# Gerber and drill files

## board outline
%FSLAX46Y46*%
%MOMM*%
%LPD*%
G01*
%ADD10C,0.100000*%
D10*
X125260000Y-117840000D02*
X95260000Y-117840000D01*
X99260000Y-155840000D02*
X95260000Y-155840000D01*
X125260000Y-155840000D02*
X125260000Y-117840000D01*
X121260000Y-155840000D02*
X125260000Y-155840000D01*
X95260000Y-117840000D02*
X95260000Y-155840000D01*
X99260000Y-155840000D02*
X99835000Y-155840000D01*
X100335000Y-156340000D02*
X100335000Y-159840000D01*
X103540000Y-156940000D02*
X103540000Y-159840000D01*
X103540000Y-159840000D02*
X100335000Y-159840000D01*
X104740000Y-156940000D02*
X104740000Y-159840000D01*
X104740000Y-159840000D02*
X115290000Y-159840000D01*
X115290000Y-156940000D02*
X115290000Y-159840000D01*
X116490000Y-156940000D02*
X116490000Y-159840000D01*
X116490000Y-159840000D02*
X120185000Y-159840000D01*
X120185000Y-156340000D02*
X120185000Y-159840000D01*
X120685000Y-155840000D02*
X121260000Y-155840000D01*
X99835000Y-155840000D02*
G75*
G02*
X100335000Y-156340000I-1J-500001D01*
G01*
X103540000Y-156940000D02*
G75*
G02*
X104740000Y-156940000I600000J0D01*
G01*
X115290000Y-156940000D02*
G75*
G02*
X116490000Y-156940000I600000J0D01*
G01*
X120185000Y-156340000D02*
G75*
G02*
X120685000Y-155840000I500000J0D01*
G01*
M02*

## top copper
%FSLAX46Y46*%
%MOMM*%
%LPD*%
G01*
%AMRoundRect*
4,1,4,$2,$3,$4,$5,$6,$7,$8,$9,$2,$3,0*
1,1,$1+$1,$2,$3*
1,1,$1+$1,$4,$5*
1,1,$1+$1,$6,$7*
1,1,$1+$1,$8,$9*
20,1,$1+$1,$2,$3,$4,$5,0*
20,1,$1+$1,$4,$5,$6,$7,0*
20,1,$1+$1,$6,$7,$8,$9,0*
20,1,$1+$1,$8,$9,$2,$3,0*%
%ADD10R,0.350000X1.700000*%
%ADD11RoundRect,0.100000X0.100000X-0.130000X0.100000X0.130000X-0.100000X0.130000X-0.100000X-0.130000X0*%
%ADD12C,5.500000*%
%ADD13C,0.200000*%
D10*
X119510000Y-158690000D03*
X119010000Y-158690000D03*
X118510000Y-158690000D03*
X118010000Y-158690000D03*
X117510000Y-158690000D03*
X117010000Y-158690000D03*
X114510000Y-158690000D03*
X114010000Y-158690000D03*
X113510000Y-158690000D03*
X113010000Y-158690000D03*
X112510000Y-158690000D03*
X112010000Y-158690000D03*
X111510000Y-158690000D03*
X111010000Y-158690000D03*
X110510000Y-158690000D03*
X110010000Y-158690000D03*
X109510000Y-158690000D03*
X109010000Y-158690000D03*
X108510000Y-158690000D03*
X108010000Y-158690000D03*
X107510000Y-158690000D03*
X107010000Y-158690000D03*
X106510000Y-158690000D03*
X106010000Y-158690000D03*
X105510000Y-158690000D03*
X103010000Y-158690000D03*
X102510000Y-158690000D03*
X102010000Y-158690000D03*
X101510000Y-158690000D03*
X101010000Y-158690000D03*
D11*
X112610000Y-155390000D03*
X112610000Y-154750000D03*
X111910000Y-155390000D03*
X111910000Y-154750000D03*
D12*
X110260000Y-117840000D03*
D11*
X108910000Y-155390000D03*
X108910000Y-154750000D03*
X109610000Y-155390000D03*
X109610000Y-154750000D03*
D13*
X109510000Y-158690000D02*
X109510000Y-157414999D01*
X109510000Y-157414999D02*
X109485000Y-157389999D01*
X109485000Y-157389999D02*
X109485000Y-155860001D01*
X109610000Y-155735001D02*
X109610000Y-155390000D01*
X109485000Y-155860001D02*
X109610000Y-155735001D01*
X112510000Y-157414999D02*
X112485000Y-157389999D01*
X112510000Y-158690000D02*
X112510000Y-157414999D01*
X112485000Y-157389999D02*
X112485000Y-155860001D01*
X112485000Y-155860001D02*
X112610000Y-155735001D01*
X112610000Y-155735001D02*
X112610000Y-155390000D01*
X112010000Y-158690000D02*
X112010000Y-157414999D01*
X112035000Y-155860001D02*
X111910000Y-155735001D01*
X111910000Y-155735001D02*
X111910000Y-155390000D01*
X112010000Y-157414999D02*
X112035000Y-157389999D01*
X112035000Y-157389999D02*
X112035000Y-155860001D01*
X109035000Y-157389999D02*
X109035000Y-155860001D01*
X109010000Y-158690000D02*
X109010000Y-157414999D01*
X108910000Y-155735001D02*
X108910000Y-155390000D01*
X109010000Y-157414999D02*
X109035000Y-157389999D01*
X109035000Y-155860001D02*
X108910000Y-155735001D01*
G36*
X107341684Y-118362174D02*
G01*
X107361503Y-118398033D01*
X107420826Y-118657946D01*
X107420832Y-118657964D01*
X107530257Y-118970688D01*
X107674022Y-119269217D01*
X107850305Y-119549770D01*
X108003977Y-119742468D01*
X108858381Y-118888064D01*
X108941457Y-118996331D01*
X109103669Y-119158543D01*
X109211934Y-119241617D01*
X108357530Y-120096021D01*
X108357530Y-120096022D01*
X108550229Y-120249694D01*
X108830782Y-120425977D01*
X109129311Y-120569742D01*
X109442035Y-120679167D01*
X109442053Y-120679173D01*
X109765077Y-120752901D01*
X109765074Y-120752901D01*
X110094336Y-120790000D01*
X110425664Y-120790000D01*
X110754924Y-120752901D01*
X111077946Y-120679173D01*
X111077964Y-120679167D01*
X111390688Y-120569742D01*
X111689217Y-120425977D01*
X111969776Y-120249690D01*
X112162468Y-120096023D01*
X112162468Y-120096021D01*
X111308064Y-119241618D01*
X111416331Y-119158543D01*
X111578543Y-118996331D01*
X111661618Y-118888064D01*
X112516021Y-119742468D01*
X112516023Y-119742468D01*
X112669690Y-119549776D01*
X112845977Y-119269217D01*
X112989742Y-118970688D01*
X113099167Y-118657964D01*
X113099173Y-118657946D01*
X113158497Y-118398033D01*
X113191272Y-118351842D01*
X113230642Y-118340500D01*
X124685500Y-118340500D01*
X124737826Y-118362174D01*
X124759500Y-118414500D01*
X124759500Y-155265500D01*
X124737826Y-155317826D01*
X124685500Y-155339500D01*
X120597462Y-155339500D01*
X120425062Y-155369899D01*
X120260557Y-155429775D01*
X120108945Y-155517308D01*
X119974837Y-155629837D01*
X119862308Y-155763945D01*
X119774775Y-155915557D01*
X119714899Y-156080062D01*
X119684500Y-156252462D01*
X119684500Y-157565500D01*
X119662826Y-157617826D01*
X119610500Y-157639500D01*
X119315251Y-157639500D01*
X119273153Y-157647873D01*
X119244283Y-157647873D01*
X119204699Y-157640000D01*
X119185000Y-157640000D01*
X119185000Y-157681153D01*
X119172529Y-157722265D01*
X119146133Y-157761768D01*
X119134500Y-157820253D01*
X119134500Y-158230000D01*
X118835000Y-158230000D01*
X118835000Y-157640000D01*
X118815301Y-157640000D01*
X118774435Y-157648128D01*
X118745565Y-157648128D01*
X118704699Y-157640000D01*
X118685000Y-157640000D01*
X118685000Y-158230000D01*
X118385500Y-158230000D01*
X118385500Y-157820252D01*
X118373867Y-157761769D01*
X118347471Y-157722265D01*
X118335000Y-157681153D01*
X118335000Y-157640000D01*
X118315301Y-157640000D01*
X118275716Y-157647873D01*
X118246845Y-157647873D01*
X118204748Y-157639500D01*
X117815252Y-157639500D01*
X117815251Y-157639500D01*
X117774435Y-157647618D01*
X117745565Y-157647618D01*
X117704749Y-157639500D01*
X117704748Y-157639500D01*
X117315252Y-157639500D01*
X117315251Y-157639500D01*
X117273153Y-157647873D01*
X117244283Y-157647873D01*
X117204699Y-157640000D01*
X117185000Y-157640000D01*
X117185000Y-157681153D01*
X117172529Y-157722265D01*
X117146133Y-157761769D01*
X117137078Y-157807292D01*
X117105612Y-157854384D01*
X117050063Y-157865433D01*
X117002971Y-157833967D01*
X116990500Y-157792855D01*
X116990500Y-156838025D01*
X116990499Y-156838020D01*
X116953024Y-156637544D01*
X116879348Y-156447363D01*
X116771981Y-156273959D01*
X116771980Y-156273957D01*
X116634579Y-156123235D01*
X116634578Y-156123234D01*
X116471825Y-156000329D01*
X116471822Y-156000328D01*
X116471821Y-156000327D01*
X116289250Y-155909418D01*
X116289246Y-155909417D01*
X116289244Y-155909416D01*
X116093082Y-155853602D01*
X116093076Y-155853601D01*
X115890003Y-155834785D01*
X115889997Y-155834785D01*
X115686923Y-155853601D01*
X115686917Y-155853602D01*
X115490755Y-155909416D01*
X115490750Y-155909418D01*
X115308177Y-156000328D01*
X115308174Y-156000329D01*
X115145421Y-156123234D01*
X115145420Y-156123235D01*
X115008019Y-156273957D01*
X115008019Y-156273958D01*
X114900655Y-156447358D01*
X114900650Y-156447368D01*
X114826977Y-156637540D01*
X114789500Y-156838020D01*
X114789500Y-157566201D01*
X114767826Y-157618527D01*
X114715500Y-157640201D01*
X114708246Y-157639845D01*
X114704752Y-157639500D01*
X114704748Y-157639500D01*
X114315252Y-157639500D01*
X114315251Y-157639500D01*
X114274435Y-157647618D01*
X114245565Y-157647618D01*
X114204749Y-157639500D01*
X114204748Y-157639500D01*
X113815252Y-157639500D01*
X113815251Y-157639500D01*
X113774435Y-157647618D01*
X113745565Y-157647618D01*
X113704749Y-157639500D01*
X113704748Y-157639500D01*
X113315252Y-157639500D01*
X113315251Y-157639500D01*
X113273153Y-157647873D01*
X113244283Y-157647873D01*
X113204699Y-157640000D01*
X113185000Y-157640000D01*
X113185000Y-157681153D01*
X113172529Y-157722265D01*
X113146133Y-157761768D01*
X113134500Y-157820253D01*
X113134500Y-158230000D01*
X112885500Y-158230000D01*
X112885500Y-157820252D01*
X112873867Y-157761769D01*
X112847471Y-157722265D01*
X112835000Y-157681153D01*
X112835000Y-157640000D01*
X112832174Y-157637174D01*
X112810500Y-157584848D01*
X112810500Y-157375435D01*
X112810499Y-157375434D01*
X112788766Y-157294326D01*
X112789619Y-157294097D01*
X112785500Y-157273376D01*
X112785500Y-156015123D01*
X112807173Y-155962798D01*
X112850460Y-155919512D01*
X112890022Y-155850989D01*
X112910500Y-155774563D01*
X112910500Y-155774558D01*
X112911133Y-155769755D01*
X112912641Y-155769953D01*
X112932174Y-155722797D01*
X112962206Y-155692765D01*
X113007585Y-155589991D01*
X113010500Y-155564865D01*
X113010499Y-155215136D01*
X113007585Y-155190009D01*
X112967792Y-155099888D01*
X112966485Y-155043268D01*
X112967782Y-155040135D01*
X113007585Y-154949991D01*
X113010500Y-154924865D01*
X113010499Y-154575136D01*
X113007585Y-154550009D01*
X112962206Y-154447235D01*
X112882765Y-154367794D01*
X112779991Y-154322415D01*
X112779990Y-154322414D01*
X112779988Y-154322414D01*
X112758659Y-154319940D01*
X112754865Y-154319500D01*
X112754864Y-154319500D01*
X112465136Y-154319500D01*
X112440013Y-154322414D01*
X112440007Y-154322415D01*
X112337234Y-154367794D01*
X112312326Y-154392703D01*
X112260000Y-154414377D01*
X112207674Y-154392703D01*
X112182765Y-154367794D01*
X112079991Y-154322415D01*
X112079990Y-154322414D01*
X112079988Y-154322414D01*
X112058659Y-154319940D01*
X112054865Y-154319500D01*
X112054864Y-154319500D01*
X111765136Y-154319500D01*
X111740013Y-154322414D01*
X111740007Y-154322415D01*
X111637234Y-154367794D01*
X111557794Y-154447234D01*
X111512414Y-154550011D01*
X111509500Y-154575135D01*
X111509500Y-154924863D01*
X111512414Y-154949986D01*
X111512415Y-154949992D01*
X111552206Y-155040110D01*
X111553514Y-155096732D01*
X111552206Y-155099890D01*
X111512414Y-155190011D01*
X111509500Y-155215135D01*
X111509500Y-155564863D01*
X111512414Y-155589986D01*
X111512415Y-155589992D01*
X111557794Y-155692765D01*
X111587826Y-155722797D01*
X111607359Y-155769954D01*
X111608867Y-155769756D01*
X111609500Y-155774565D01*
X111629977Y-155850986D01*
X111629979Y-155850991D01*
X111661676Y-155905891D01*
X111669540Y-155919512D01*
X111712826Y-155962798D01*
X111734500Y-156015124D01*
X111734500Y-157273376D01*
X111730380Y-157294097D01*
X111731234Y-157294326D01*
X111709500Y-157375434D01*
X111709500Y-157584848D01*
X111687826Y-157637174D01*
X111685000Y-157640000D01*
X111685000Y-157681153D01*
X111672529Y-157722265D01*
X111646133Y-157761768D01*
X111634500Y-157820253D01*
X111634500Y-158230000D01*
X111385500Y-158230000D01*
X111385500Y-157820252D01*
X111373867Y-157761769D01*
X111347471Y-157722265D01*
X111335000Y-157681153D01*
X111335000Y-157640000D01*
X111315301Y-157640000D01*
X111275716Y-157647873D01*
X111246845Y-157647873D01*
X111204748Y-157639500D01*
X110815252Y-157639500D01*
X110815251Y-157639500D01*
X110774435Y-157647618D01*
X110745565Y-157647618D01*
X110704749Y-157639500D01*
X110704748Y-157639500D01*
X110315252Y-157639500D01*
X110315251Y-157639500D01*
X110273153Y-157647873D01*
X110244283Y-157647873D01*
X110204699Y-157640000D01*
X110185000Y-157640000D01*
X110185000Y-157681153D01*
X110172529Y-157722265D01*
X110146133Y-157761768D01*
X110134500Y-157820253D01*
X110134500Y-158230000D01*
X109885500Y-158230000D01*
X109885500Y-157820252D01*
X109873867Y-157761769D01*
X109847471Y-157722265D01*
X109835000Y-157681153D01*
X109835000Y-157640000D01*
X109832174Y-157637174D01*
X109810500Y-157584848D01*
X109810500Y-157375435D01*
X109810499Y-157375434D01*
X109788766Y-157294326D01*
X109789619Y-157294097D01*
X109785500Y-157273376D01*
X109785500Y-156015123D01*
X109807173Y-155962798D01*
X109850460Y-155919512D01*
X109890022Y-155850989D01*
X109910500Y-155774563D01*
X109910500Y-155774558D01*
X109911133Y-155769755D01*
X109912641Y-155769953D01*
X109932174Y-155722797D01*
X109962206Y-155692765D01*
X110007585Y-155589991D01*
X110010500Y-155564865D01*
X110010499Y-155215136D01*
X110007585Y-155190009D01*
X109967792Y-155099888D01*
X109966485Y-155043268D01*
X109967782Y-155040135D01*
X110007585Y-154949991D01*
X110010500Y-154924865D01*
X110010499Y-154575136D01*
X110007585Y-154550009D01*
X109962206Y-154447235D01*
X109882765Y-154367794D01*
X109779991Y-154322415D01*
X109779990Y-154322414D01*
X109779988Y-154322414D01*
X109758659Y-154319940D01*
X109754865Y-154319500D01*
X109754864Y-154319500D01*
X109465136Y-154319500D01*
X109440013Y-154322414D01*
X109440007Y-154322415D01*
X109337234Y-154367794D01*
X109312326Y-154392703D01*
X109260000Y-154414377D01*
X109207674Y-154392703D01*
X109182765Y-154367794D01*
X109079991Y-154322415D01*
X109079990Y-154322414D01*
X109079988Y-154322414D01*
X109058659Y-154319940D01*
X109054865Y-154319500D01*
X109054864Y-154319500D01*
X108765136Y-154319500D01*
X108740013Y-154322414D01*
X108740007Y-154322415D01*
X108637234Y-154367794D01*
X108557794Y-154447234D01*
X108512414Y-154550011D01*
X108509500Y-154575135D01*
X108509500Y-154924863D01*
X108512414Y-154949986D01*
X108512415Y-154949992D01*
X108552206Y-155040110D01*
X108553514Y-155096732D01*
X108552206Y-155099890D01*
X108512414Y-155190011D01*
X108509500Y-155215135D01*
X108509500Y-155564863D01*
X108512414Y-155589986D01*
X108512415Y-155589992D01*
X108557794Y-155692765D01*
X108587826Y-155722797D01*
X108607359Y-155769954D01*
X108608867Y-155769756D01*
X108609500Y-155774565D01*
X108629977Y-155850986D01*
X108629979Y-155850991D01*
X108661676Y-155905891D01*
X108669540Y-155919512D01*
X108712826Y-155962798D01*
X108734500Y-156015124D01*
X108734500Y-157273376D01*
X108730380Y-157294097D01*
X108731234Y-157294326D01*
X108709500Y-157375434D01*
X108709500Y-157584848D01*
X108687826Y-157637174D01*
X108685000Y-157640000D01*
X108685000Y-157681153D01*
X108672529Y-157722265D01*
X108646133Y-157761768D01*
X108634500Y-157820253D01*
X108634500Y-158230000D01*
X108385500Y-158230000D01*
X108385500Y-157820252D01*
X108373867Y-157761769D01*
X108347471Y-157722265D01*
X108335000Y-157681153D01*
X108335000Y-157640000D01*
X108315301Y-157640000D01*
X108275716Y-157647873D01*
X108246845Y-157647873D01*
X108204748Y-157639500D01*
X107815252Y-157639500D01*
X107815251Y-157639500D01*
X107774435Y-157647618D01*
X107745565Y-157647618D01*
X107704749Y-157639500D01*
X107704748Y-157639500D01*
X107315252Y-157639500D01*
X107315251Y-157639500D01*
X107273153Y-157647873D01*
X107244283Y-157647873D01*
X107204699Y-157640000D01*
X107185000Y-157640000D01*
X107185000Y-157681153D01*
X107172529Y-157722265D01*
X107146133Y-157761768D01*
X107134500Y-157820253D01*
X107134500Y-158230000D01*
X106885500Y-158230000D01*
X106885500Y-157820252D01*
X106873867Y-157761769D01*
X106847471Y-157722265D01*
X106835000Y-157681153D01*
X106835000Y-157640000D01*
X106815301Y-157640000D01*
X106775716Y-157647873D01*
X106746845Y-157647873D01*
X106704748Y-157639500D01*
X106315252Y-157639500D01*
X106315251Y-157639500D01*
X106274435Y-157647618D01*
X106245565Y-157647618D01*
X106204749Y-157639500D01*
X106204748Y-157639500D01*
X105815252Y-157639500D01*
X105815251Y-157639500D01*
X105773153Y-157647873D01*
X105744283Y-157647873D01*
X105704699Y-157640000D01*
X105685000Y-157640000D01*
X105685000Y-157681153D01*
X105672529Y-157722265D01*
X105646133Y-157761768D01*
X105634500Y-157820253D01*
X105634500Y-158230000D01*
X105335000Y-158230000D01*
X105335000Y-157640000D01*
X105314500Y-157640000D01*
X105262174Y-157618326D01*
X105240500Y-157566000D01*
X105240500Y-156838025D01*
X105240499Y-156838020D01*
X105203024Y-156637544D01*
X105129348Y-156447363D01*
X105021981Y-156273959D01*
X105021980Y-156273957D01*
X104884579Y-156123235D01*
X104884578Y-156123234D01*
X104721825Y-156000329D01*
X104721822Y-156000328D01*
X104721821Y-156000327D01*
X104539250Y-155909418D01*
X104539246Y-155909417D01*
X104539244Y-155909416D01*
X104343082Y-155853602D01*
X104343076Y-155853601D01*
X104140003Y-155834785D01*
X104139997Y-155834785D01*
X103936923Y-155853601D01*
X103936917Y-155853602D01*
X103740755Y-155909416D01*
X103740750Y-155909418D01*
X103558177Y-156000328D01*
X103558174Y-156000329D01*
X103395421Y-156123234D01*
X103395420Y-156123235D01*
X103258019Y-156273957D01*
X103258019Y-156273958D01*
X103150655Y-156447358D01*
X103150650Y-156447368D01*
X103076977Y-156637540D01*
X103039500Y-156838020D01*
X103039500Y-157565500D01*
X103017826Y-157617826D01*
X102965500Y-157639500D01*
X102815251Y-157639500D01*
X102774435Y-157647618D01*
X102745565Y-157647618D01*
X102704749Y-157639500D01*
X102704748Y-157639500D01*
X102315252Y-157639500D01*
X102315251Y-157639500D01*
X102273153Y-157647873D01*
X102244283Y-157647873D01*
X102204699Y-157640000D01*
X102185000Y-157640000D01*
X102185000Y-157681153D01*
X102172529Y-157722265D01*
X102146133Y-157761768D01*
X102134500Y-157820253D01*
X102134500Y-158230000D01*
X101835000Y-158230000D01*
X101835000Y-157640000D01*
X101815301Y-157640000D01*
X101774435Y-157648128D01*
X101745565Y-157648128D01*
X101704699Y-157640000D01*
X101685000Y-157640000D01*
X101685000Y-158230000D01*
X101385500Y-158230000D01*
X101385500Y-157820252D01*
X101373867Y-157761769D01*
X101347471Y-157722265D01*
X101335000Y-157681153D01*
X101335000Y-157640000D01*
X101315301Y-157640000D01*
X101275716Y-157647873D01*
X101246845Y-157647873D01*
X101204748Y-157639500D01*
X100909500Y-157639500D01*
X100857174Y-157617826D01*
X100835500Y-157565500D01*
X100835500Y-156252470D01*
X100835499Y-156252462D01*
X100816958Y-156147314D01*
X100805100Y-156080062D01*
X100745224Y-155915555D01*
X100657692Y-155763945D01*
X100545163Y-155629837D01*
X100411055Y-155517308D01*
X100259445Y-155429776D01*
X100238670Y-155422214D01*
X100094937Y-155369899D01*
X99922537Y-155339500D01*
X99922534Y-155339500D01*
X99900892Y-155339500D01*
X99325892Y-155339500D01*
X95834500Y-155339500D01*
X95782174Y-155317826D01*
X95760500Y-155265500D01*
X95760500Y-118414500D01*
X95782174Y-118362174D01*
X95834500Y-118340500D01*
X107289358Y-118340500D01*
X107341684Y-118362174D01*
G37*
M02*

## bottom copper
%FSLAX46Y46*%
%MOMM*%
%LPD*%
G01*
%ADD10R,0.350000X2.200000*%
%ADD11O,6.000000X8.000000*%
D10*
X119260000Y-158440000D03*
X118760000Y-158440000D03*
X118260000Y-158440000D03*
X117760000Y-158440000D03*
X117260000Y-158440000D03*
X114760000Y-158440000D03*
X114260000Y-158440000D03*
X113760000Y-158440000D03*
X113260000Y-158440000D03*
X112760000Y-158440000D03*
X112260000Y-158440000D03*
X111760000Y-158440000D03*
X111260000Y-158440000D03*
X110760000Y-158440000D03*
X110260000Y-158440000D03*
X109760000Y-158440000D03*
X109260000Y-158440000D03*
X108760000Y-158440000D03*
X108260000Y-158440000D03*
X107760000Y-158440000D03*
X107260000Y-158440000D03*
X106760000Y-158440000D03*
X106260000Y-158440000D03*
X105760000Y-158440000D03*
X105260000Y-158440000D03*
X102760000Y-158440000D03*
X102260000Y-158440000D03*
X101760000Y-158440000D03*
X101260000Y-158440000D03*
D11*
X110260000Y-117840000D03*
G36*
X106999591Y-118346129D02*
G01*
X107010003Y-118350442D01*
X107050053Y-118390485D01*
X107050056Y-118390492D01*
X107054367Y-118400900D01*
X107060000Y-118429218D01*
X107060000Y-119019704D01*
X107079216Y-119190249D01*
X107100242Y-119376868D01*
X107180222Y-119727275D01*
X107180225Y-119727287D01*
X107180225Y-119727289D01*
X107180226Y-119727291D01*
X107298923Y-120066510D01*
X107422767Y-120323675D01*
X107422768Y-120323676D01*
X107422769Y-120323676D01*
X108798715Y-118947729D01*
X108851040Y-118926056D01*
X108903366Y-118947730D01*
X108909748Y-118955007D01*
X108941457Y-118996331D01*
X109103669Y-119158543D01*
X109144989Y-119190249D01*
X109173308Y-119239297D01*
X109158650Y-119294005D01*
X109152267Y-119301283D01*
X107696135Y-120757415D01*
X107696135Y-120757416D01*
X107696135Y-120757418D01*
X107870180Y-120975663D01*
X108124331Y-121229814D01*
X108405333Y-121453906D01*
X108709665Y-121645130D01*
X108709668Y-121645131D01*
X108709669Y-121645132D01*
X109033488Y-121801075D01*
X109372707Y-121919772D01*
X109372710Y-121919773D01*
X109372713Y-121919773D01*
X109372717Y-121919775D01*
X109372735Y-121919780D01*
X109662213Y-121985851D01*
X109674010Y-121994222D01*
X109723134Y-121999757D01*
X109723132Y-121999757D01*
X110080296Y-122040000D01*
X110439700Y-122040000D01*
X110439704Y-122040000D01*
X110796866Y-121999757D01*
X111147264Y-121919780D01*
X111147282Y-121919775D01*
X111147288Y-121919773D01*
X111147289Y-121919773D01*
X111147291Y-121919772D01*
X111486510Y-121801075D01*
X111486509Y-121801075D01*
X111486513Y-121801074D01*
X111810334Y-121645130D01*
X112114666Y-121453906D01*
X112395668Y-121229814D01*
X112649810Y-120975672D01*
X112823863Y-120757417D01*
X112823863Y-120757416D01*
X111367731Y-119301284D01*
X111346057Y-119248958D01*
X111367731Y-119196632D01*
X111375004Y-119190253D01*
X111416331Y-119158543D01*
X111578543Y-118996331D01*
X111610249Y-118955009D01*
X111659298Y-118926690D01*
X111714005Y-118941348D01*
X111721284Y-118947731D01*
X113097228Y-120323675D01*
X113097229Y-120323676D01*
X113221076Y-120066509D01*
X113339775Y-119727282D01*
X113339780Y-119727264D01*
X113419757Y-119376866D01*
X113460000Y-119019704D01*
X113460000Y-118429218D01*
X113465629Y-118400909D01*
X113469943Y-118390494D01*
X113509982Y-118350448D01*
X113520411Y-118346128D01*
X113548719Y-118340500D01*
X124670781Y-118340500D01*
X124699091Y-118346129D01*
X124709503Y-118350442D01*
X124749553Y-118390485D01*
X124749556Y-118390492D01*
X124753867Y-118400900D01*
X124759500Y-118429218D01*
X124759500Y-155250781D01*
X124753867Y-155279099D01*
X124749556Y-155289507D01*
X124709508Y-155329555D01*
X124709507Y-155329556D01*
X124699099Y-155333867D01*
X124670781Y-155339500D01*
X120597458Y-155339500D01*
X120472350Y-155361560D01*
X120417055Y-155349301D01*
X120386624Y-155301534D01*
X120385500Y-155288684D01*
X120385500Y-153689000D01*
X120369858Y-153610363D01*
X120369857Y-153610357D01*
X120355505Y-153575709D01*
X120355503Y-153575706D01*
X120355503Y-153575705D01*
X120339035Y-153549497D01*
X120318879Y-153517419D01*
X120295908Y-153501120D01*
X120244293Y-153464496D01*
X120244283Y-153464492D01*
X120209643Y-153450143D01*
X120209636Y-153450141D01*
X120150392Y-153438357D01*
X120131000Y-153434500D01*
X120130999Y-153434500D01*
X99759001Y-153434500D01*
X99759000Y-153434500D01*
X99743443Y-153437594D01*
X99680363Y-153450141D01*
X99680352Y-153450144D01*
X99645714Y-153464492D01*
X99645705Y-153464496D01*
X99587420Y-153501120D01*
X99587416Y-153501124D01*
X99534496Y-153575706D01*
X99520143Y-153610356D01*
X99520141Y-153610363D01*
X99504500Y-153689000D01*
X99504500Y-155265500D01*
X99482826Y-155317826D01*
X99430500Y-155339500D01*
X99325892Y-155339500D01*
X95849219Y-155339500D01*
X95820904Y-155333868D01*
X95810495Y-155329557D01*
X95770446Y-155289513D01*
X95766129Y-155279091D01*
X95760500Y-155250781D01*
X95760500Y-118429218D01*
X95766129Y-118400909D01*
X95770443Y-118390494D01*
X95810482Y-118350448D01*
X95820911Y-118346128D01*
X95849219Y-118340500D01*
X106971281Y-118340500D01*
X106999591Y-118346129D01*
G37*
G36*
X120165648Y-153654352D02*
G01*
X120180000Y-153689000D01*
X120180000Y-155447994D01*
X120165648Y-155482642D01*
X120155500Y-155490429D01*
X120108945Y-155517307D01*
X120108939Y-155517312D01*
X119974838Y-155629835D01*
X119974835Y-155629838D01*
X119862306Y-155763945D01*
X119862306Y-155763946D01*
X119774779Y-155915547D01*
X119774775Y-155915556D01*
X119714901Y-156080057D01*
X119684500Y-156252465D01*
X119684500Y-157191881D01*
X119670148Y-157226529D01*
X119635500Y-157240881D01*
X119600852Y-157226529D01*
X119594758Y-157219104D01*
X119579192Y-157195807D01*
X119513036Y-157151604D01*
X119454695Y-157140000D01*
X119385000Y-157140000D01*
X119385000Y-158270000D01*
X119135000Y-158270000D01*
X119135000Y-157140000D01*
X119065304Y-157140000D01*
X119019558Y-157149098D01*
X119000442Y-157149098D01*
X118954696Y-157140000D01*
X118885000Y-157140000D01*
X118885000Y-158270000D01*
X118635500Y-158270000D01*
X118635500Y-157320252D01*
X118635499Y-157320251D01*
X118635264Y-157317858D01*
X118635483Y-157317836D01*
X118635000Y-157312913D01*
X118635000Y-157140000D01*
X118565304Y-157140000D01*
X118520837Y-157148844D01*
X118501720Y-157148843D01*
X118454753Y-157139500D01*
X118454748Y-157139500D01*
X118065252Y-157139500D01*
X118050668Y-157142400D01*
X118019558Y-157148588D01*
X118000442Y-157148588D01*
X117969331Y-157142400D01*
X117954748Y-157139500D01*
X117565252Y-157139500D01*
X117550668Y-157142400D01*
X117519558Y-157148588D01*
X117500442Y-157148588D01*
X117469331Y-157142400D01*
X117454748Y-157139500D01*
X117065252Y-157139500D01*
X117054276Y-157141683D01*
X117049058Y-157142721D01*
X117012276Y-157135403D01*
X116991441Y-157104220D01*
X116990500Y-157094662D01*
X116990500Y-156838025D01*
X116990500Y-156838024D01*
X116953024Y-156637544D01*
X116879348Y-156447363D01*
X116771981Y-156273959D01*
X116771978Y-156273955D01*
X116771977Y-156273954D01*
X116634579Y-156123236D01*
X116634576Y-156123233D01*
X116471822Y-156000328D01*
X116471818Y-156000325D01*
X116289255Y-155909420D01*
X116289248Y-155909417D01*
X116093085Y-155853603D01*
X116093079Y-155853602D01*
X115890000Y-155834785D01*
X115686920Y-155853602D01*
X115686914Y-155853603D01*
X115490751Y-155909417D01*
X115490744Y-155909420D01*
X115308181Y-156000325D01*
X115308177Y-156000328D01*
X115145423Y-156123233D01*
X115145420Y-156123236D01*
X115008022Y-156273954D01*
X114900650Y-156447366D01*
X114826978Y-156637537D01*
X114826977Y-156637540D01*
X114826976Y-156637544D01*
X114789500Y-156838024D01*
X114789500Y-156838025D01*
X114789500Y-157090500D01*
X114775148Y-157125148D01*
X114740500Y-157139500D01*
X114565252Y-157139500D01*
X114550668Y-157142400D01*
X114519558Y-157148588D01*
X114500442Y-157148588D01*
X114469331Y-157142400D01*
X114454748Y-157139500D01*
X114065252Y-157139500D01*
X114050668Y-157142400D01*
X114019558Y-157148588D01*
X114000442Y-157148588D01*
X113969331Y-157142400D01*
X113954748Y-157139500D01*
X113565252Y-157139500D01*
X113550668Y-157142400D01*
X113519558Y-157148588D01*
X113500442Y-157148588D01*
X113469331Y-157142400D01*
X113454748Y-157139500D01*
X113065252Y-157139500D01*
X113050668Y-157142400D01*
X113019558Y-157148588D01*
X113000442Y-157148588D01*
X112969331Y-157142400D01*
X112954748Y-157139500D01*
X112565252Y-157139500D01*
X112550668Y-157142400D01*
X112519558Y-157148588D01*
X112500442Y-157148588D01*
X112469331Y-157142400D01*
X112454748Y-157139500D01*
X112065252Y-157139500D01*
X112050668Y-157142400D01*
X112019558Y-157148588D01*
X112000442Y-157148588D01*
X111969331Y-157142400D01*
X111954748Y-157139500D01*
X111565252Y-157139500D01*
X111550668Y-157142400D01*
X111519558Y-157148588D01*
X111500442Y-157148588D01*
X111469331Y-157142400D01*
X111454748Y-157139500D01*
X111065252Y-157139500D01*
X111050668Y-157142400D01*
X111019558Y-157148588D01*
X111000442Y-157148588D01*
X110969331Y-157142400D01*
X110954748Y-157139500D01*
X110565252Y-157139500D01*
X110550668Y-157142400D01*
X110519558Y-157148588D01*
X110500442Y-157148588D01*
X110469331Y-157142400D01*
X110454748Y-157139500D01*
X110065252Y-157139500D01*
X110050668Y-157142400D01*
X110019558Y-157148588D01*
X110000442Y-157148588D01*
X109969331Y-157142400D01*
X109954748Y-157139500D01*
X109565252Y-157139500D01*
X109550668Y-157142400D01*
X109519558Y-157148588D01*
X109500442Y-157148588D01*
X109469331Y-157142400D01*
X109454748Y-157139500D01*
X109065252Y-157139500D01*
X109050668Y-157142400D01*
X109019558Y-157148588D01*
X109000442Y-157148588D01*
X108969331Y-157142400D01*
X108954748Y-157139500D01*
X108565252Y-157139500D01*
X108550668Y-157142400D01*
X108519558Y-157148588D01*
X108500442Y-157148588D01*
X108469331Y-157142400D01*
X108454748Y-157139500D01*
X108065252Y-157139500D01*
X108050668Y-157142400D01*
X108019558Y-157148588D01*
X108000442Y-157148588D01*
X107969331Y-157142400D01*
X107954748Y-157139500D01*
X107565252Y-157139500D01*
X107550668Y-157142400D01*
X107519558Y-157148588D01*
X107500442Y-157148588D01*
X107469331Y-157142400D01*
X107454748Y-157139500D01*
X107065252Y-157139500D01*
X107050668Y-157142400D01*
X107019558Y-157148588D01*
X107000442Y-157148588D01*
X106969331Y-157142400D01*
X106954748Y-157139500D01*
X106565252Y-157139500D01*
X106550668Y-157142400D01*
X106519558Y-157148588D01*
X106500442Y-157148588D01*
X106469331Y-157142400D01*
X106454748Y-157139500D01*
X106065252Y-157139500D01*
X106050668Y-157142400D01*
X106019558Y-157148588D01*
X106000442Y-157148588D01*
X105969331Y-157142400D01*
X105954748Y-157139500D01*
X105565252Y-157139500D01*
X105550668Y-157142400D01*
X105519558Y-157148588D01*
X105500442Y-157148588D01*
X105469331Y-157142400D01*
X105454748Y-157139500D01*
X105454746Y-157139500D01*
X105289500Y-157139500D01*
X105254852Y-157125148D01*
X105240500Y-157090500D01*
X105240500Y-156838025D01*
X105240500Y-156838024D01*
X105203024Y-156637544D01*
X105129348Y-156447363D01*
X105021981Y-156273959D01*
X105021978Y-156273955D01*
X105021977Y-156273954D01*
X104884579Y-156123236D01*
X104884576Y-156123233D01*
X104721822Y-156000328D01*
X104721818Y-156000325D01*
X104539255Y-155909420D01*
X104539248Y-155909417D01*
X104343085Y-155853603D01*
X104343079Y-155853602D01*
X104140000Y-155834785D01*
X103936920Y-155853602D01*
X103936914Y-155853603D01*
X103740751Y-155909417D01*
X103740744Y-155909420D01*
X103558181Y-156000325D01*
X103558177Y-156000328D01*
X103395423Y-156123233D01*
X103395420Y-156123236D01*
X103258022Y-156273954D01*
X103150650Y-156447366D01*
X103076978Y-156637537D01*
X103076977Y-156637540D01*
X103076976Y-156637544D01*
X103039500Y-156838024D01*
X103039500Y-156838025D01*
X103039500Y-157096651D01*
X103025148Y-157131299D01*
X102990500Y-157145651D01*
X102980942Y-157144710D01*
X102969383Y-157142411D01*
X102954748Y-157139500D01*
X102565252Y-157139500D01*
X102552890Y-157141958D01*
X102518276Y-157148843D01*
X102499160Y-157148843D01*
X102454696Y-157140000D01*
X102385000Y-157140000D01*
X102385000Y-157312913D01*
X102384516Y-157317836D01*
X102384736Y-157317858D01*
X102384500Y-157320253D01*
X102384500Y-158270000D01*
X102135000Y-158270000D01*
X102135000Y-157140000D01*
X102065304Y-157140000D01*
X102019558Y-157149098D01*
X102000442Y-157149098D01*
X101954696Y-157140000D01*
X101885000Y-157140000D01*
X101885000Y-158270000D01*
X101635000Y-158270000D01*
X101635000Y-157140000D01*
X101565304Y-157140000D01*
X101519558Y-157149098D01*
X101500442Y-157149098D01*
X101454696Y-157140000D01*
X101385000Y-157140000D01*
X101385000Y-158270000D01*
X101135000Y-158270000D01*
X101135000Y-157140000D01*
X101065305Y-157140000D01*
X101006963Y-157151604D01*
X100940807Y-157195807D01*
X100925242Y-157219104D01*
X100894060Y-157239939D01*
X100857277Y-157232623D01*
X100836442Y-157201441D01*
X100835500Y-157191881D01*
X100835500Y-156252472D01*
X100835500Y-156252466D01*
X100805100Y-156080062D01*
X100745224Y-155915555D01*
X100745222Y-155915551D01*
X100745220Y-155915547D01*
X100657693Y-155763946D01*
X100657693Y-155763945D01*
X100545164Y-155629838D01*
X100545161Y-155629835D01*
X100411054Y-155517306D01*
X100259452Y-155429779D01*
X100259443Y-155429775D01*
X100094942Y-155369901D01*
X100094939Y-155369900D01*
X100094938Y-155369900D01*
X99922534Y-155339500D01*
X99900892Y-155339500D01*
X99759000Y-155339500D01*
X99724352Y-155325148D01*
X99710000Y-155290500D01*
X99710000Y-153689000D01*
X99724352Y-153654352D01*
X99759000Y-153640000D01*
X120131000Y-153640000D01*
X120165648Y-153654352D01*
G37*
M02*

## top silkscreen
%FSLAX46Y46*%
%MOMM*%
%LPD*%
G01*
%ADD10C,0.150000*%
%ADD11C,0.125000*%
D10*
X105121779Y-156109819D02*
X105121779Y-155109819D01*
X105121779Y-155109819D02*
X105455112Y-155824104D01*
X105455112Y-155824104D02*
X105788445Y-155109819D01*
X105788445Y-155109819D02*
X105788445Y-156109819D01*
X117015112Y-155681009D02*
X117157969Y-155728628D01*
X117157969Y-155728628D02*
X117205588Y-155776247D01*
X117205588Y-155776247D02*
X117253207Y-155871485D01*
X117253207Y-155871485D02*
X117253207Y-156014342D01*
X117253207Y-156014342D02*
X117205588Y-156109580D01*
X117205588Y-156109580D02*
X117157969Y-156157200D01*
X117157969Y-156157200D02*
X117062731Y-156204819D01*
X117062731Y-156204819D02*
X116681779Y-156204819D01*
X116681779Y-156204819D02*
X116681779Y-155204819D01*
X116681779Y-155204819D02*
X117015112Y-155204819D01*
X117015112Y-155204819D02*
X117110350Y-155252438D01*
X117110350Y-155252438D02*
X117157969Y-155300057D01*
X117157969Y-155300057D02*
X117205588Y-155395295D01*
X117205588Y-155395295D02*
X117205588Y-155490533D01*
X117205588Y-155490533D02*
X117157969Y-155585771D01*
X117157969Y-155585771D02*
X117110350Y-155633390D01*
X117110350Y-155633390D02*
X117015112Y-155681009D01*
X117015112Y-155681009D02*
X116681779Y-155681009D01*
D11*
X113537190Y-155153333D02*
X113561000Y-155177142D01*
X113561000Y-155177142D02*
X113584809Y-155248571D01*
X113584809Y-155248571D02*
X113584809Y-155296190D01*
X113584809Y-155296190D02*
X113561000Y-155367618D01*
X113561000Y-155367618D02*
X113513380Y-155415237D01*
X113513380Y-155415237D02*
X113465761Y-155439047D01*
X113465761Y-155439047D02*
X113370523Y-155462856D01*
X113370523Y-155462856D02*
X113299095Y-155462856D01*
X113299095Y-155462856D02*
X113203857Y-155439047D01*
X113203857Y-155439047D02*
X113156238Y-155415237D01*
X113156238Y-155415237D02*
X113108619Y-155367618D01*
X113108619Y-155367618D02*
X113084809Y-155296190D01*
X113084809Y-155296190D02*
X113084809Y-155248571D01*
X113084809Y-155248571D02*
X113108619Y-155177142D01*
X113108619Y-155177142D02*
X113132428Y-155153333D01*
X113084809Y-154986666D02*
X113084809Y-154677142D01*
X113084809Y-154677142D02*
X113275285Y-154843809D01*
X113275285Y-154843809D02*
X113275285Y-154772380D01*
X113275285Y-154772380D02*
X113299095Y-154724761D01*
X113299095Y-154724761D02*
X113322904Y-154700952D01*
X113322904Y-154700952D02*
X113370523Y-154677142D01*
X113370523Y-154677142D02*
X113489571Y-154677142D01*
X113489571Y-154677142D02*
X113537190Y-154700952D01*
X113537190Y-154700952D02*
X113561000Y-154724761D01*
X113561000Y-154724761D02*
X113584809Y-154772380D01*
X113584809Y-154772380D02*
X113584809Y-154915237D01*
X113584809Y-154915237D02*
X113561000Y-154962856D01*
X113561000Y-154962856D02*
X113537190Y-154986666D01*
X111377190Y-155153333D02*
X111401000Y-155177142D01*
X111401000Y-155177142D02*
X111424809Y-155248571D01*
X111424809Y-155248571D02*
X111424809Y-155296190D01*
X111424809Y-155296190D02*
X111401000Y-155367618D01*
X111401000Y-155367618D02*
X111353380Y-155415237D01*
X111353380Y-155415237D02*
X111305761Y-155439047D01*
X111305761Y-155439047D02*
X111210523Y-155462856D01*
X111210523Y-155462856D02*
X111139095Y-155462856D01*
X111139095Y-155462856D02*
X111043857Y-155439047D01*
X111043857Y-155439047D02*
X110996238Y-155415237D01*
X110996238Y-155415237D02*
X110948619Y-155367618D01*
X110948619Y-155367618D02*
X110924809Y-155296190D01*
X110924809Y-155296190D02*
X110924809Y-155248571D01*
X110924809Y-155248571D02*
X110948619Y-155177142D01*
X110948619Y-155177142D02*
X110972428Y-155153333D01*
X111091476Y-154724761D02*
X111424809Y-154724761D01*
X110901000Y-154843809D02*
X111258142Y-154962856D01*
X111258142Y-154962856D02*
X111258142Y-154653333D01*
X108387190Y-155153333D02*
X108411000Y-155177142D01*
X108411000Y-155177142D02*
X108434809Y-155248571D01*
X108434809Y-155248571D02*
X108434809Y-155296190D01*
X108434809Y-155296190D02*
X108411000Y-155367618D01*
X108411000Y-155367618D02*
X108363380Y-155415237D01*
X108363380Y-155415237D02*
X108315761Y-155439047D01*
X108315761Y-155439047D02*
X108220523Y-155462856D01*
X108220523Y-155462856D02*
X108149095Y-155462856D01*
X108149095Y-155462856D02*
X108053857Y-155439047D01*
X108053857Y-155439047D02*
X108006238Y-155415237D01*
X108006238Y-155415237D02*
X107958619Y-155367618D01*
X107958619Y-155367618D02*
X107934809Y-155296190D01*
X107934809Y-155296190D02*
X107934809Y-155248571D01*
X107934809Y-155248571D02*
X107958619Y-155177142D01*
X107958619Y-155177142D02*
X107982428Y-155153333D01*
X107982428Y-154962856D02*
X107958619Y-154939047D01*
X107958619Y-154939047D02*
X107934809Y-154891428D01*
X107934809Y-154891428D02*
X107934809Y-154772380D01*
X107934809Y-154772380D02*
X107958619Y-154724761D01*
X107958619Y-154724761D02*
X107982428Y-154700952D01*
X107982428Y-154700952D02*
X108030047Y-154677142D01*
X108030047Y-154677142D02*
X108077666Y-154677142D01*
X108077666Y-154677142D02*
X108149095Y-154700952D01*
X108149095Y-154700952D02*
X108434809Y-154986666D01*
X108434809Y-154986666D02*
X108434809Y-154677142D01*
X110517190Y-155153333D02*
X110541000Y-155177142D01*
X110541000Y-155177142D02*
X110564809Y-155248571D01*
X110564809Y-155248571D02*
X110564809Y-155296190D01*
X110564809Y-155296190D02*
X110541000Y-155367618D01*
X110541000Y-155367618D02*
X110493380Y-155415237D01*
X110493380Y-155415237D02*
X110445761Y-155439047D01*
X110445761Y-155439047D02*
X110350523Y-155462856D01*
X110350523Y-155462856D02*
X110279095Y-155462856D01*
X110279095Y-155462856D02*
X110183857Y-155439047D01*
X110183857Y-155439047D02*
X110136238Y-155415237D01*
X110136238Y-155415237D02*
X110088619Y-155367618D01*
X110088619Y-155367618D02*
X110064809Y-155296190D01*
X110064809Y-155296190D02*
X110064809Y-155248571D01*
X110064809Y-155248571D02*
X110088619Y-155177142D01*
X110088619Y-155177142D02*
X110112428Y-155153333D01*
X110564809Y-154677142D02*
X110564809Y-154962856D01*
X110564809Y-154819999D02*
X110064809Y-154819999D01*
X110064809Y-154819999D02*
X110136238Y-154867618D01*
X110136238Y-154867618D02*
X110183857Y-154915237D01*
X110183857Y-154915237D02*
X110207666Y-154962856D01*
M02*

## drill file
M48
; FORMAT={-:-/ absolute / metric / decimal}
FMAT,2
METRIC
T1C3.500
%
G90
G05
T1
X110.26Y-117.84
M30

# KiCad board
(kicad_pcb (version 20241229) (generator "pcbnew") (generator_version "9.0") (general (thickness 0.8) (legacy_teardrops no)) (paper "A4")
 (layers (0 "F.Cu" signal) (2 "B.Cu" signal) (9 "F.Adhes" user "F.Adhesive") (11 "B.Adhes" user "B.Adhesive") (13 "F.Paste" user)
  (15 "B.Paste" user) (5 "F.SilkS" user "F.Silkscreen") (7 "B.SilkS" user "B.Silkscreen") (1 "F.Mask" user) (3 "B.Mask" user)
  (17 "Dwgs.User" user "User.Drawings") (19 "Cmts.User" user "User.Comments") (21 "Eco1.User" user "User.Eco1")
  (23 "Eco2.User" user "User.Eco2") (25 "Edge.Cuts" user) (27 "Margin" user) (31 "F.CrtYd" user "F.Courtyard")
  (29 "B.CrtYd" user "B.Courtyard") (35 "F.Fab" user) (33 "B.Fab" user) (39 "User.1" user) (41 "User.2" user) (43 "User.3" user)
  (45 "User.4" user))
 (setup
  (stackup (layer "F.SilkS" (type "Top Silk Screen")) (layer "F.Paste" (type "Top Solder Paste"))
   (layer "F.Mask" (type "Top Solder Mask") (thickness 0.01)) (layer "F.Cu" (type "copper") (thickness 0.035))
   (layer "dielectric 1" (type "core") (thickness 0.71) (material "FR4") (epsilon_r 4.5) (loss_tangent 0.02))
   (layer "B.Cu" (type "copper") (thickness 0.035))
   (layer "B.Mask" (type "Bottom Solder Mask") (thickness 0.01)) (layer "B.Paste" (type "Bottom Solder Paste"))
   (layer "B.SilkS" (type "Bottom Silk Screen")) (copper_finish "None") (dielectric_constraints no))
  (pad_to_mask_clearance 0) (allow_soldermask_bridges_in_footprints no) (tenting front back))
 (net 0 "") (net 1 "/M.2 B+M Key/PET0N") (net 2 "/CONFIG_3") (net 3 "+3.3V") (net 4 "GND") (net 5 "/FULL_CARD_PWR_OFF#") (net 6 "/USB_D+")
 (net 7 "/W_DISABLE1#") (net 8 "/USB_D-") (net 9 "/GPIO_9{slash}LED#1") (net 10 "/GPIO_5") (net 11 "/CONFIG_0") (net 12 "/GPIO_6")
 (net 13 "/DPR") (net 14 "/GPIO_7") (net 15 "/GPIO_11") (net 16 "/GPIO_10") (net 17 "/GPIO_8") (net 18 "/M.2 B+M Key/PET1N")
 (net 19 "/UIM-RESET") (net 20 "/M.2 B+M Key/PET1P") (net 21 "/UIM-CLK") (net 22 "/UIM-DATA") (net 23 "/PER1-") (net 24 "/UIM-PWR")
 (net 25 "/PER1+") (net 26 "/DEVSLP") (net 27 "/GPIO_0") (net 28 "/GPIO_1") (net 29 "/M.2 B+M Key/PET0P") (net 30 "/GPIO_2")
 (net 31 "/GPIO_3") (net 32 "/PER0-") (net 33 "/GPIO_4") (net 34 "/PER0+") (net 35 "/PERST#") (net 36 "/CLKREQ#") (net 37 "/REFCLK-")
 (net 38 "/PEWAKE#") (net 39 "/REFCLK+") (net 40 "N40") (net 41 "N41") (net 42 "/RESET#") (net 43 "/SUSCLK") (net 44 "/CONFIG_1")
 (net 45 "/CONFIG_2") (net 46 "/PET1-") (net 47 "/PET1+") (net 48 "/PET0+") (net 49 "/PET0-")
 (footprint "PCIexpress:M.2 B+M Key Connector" (layer "F.Cu") (at 110.26 158.73)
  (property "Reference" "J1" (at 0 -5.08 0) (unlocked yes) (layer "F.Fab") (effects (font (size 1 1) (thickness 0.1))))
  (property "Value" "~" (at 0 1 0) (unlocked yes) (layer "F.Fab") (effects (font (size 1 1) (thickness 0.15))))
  (fp_line (start -11 -2.89) (end -10.425 -2.89) (stroke (width 0.1) (type default)) (layer "Edge.Cuts") (net 1))
  (fp_line (start -9.925 -2.39) (end -9.925 1.11) (stroke (width 0.1) (type default)) (layer "Edge.Cuts") (net 1))
  (fp_line (start -6.72 -1.79) (end -6.72 1.11) (stroke (width 0.1) (type default)) (layer "Edge.Cuts") (net 1))
  (fp_line (start -6.72 1.11) (end -9.925 1.11) (stroke (width 0.1) (type default)) (layer "Edge.Cuts") (net 1))
  (fp_line (start -5.52 -1.79) (end -5.52 1.11) (stroke (width 0.1) (type default)) (layer "Edge.Cuts") (net 1))
  (fp_line (start -5.52 1.11) (end 5.03 1.11) (stroke (width 0.1) (type default)) (layer "Edge.Cuts") (net 1))
  (fp_line (start 5.03 -1.79) (end 5.03 1.11) (stroke (width 0.1) (type default)) (layer "Edge.Cuts") (net 1))
  (fp_line (start 6.23 -1.79) (end 6.23 1.11) (stroke (width 0.1) (type default)) (layer "Edge.Cuts") (net 1))
  (fp_line (start 6.23 1.11) (end 9.925 1.11) (stroke (width 0.1) (type default)) (layer "Edge.Cuts") (net 1))
  (fp_line (start 9.925 -2.39) (end 9.925 1.11) (stroke (width 0.1) (type default)) (layer "Edge.Cuts") (net 1))
  (fp_line (start 10.425 -2.89) (end 11 -2.89) (stroke (width 0.1) (type default)) (layer "Edge.Cuts") (net 1))
  (fp_arc (start -10.425 -2.89) (mid -10.071447 -2.743553) (end -9.925 -2.39) (stroke (width 0.1) (type default)) (layer "Edge.Cuts")
   (net 1))
  (fp_arc (start -6.72 -1.79) (mid -6.12 -2.39) (end -5.52 -1.79) (stroke (width 0.1) (type default)) (layer "Edge.Cuts") (net 1))
  (fp_arc (start 5.03 -1.79) (mid 5.63 -2.39) (end 6.23 -1.79) (stroke (width 0.1) (type default)) (layer "Edge.Cuts") (net 1))
  (fp_arc (start 9.925 -2.39) (mid 10.071447 -2.743553) (end 10.425 -2.89) (stroke (width 0.1) (type default)) (layer "Edge.Cuts") (net 1))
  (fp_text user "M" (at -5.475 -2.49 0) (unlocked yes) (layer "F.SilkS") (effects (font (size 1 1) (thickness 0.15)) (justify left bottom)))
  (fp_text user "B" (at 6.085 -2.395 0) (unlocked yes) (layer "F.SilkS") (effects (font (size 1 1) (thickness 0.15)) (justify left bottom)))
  (pad "1" smd rect (at 9.25 -0.04 180) (size 0.35 1.7) (layers "F.Cu") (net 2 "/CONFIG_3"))
  (pad "2" smd rect (at 9 -0.29 180) (size 0.35 2.2) (layers "B.Cu") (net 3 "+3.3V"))
  (pad "3" smd rect (at 8.75 -0.04 180) (size 0.35 1.7) (layers "F.Cu") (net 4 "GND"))
  (pad "4" smd rect (at 8.5 -0.29 180) (size 0.35 2.2) (layers "B.Cu") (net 3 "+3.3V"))
  (pad "5" smd rect (at 8.25 -0.04 180) (size 0.35 1.7) (layers "F.Cu") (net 4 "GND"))
  (pad "6" smd rect (at 8 -0.29 180) (size 0.35 2.2) (layers "B.Cu") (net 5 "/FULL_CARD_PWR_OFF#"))
  (pad "7" smd rect (at 7.75 -0.04 180) (size 0.35 1.7) (layers "F.Cu") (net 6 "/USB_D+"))
  (pad "8" smd rect (at 7.5 -0.29 180) (size 0.35 2.2) (layers "B.Cu") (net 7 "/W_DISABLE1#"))
  (pad "9" smd rect (at 7.25 -0.04 180) (size 0.35 1.7) (layers "F.Cu") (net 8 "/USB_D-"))
  (pad "10" smd rect (at 7 -0.29 180) (size 0.35 2.2) (layers "B.Cu") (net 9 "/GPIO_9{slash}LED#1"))
  (pad "11" smd rect (at 6.75 -0.04 180) (size 0.35 1.7) (layers "F.Cu") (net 4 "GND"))
  (pad "20" smd rect (at 4.5 -0.29 180) (size 0.35 2.2) (layers "B.Cu") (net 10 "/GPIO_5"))
  (pad "21" smd rect (at 4.25 -0.04 180) (size 0.35 1.7) (layers "F.Cu") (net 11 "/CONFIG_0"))
  (pad "22" smd rect (at 4 -0.29 180) (size 0.35 2.2) (layers "B.Cu") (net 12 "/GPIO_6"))
  (pad "23" smd rect (at 3.75 -0.04 180) (size 0.35 1.7) (layers "F.Cu") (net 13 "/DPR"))
  (pad "24" smd rect (at 3.5 -0.29 180) (size 0.35 2.2) (layers "B.Cu") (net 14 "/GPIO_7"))
  (pad "25" smd rect (at 3.25 -0.04 180) (size 0.35 1.7) (layers "F.Cu") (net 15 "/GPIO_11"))
  (pad "26" smd rect (at 3 -0.29 180) (size 0.35 2.2) (layers "B.Cu") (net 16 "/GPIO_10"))
  (pad "27" smd rect (at 2.75 -0.04 180) (size 0.35 1.7) (layers "F.Cu") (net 4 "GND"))
  (pad "28" smd rect (at 2.5 -0.29 180) (size 0.35 2.2) (layers "B.Cu") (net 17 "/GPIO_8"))
  (pad "29" smd rect (at 2.25 -0.04 180) (size 0.35 1.7) (layers "F.Cu") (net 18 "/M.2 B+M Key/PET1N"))
  (pad "30" smd rect (at 2 -0.29 180) (size 0.35 2.2) (layers "B.Cu") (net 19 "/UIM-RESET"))
  (pad "31" smd rect (at 1.75 -0.04 180) (size 0.35 1.7) (layers "F.Cu") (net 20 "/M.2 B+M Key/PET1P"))
  (pad "32" smd rect (at 1.5 -0.29 180) (size 0.35 2.2) (layers "B.Cu") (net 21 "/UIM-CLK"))
  (pad "33" smd rect (at 1.25 -0.04 180) (size 0.35 1.7) (layers "F.Cu") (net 4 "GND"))
  (pad "34" smd rect (at 1 -0.29 180) (size 0.35 2.2) (layers "B.Cu") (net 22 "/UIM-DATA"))
  (pad "35" smd rect (at 0.75 -0.04 180) (size 0.35 1.7) (layers "F.Cu") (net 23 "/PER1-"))
  (pad "36" smd rect (at 0.5 -0.29 180) (size 0.35 2.2) (layers "B.Cu") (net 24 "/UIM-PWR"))
  (pad "37" smd rect (at 0.25 -0.04 180) (size 0.35 1.7) (layers "F.Cu") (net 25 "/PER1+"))
  (pad "38" smd rect (at 0 -0.29 180) (size 0.35 2.2) (layers "B.Cu") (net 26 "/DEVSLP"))
  (pad "39" smd rect (at -0.25 -0.04 180) (size 0.35 1.7) (layers "F.Cu") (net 4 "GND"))
  (pad "40" smd rect (at -0.5 -0.29 180) (size 0.35 2.2) (layers "B.Cu") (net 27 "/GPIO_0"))
  (pad "41" smd rect (at -0.75 -0.04 180) (size 0.35 1.7) (layers "F.Cu") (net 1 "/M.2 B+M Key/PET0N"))
  (pad "42" smd rect (at -1 -0.29 180) (size 0.35 2.2) (layers "B.Cu") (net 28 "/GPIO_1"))
  (pad "43" smd rect (at -1.25 -0.04 180) (size 0.35 1.7) (layers "F.Cu") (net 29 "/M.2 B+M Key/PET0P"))
  (pad "44" smd rect (at -1.5 -0.29 180) (size 0.35 2.2) (layers "B.Cu") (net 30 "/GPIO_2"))
  (pad "45" smd rect (at -1.75 -0.04 180) (size 0.35 1.7) (layers "F.Cu") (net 4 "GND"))
  (pad "46" smd rect (at -2 -0.29 180) (size 0.35 2.2) (layers "B.Cu") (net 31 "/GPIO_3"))
  (pad "47" smd rect (at -2.25 -0.04 180) (size 0.35 1.7) (layers "F.Cu") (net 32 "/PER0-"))
  (pad "48" smd rect (at -2.5 -0.29 180) (size 0.35 2.2) (layers "B.Cu") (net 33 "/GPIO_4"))
  (pad "49" smd rect (at -2.75 -0.04 180) (size 0.35 1.7) (layers "F.Cu") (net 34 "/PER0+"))
  (pad "50" smd rect (at -3 -0.29 180) (size 0.35 2.2) (layers "B.Cu") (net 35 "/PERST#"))
  (pad "51" smd rect (at -3.25 -0.04 180) (size 0.35 1.7) (layers "F.Cu") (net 4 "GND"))
  (pad "52" smd rect (at -3.5 -0.29 180) (size 0.35 2.2) (layers "B.Cu") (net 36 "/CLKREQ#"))
  (pad "53" smd rect (at -3.75 -0.04 180) (size 0.35 1.7) (layers "F.Cu") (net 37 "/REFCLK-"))
  (pad "54" smd rect (at -4 -0.29 180) (size 0.35 2.2) (layers "B.Cu") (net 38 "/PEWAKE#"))
  (pad "55" smd rect (at -4.25 -0.04 180) (size 0.35 1.7) (layers "F.Cu") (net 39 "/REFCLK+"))
  (pad "56" smd rect (at -4.5 -0.29 180) (size 0.35 2.2) (layers "B.Cu") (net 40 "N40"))
  (pad "57" smd rect (at -4.75 -0.04 180) (size 0.35 1.7) (layers "F.Cu") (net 4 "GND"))
  (pad "58" smd rect (at -5 -0.29 180) (size 0.35 2.2) (layers "B.Cu") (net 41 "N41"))
  (pad "67" smd rect (at -7.25 -0.04 180) (size 0.35 1.7) (layers "F.Cu") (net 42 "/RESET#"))
  (pad "68" smd rect (at -7.5 -0.29 180) (size 0.35 2.2) (layers "B.Cu") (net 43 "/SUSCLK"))
  (pad "69" smd rect (at -7.75 -0.04 180) (size 0.35 1.7) (layers "F.Cu") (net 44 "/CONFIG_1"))
  (pad "70" smd rect (at -8 -0.29 180) (size 0.35 2.2) (layers "B.Cu") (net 3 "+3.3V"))
  (pad "71" smd rect (at -8.25 -0.04 180) (size 0.35 1.7) (layers "F.Cu") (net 4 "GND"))
  (pad "72" smd rect (at -8.5 -0.29 180) (size 0.35 2.2) (layers "B.Cu") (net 3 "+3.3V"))
  (pad "73" smd rect (at -8.75 -0.04 180) (size 0.35 1.7) (layers "F.Cu") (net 4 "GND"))
  (pad "74" smd rect (at -9 -0.29 180) (size 0.35 2.2) (layers "B.Cu") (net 3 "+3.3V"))
  (pad "75" smd rect (at -9.25 -0.04 180) (size 0.35 1.7) (layers "F.Cu") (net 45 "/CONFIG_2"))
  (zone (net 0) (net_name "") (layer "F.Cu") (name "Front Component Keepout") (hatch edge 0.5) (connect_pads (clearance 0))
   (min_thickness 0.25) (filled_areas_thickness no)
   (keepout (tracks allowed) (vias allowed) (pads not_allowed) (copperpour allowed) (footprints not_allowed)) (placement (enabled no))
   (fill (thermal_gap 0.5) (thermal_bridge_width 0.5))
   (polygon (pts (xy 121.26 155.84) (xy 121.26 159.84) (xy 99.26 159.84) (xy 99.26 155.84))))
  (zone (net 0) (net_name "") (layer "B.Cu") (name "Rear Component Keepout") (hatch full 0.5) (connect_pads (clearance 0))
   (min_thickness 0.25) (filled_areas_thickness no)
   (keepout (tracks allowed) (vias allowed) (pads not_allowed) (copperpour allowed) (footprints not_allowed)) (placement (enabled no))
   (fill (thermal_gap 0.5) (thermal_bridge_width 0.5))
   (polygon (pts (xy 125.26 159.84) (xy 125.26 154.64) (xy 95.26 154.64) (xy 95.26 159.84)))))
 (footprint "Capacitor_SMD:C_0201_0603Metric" (layer "F.Cu") (at 112.61 155.07 90)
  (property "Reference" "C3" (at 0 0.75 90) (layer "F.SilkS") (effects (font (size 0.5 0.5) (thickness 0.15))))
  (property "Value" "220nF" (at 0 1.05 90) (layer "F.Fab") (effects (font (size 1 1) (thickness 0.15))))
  (pad "" smd roundrect (at -0.345 0 90) (size 0.318 0.36) (layers "F.Paste") (roundrect_rratio 0.25))
  (pad "" smd roundrect (at 0.345 0 90) (size 0.318 0.36) (layers "F.Paste") (roundrect_rratio 0.25))
  (pad "1" smd roundrect (at -0.32 0 90) (size 0.46 0.4) (layers "F.Cu" "F.Mask") (roundrect_rratio 0.25) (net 18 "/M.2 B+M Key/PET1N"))
  (pad "2" smd roundrect (at 0.32 0 90) (size 0.46 0.4) (layers "F.Cu" "F.Mask") (roundrect_rratio 0.25) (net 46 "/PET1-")))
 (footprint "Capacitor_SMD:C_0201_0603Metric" (layer "F.Cu") (at 111.91 155.07 90)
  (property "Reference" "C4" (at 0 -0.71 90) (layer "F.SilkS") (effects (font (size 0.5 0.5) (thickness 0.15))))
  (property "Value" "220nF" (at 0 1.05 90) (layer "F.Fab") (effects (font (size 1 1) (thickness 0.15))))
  (pad "" smd roundrect (at -0.345 0 90) (size 0.318 0.36) (layers "F.Paste") (roundrect_rratio 0.25))
  (pad "" smd roundrect (at 0.345 0 90) (size 0.318 0.36) (layers "F.Paste") (roundrect_rratio 0.25))
  (pad "1" smd roundrect (at -0.32 0 90) (size 0.46 0.4) (layers "F.Cu" "F.Mask") (roundrect_rratio 0.25) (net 20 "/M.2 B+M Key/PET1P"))
  (pad "2" smd roundrect (at 0.32 0 90) (size 0.46 0.4) (layers "F.Cu" "F.Mask") (roundrect_rratio 0.25) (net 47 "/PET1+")))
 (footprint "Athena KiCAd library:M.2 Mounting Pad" (layer "F.Cu") (at 110.26 117.84)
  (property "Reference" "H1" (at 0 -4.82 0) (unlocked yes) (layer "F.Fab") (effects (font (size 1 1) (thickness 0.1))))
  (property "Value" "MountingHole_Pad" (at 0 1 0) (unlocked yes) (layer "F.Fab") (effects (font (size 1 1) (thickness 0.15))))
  (pad "1" thru_hole circle (at 0 0) (size 5.5 5.5) (drill 3.5) (layers "*.Cu" "*.Mask") (remove_unused_layers no) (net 4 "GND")
   (padstack (mode front_inner_back)
    (layer "Inner" (shape circle) (size 5.5 5.5) (zone_connect -1))
    (layer "B.Cu" (shape oval) (size 6 8) (thermal_bridge_angle 45) (zone_connect -1)))))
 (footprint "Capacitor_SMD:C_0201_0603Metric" (layer "F.Cu") (at 108.91 155.07 90)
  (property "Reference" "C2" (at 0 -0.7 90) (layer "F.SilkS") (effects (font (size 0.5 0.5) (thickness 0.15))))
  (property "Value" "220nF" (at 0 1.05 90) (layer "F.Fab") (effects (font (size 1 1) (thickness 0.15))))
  (pad "" smd roundrect (at -0.345 0 90) (size 0.318 0.36) (layers "F.Paste") (roundrect_rratio 0.25))
  (pad "" smd roundrect (at 0.345 0 90) (size 0.318 0.36) (layers "F.Paste") (roundrect_rratio 0.25))
  (pad "1" smd roundrect (at -0.32 0 90) (size 0.46 0.4) (layers "F.Cu" "F.Mask") (roundrect_rratio 0.25) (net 29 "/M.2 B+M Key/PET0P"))
  (pad "2" smd roundrect (at 0.32 0 90) (size 0.46 0.4) (layers "F.Cu" "F.Mask") (roundrect_rratio 0.25) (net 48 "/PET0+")))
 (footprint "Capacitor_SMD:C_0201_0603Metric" (layer "F.Cu") (at 109.61 155.07 90)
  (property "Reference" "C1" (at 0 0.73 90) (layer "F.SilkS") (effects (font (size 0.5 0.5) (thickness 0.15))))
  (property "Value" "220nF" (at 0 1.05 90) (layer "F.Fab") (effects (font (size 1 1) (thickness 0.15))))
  (pad "" smd roundrect (at -0.345 0 90) (size 0.318 0.36) (layers "F.Paste") (roundrect_rratio 0.25))
  (pad "" smd roundrect (at 0.345 0 90) (size 0.318 0.36) (layers "F.Paste") (roundrect_rratio 0.25))
  (pad "1" smd roundrect (at -0.32 0 90) (size 0.46 0.4) (layers "F.Cu" "F.Mask") (roundrect_rratio 0.25) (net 1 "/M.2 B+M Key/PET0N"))
  (pad "2" smd roundrect (at 0.32 0 90) (size 0.46 0.4) (layers "F.Cu" "F.Mask") (roundrect_rratio 0.25) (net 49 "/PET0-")))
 (gr_line (start 125.26 117.84) (end 95.26 117.84) (stroke (width 0.1) (type default)) (layer "Edge.Cuts"))
 (gr_line (start 99.26 155.84) (end 95.26 155.84) (stroke (width 0.1) (type default)) (layer "Edge.Cuts"))
 (gr_line (start 125.26 155.84) (end 125.26 117.84) (stroke (width 0.1) (type default)) (layer "Edge.Cuts"))
 (gr_line (start 121.26 155.84) (end 125.26 155.84) (stroke (width 0.1) (type default)) (layer "Edge.Cuts"))
 (gr_line (start 95.26 117.84) (end 95.26 155.84) (stroke (width 0.1) (type default)) (layer "Edge.Cuts"))
 (segment (start 109.51 158.69) (end 109.51 157.414999) (width 0.2) (layer "F.Cu") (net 1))
 (segment (start 109.51 157.414999) (end 109.485 157.389999) (width 0.2) (layer "F.Cu") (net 1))
 (segment (start 109.485 157.389999) (end 109.485 155.860001) (width 0.2) (layer "F.Cu") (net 1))
 (segment (start 109.61 155.735001) (end 109.61 155.39) (width 0.2) (layer "F.Cu") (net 1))
 (segment (start 109.485 155.860001) (end 109.61 155.735001) (width 0.2) (layer "F.Cu") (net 1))
 (segment (start 112.51 157.414999) (end 112.485 157.389999) (width 0.2) (layer "F.Cu") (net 18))
 (segment (start 112.51 158.69) (end 112.51 157.414999) (width 0.2) (layer "F.Cu") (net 18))
 (segment (start 112.485 157.389999) (end 112.485 155.860001) (width 0.2) (layer "F.Cu") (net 18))
 (segment (start 112.485 155.860001) (end 112.61 155.735001) (width 0.2) (layer "F.Cu") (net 18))
 (segment (start 112.61 155.735001) (end 112.61 155.39) (width 0.2) (layer "F.Cu") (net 18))
 (segment (start 112.01 158.69) (end 112.01 157.414999) (width 0.2) (layer "F.Cu") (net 20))
 (segment (start 112.035 155.860001) (end 111.91 155.735001) (width 0.2) (layer "F.Cu") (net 20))
 (segment (start 111.91 155.735001) (end 111.91 155.39) (width 0.2) (layer "F.Cu") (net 20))
 (segment (start 112.01 157.414999) (end 112.035 157.389999) (width 0.2) (layer "F.Cu") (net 20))
 (segment (start 112.035 157.389999) (end 112.035 155.860001) (width 0.2) (layer "F.Cu") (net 20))
 (segment (start 109.035 157.389999) (end 109.035 155.860001) (width 0.2) (layer "F.Cu") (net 29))
 (segment (start 109.01 158.69) (end 109.01 157.414999) (width 0.2) (layer "F.Cu") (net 29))
 (segment (start 108.91 155.735001) (end 108.91 155.39) (width 0.2) (layer "F.Cu") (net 29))
 (segment (start 109.01 157.414999) (end 109.035 157.389999) (width 0.2) (layer "F.Cu") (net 29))
 (segment (start 109.035 155.860001) (end 108.91 155.735001) (width 0.2) (layer "F.Cu") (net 29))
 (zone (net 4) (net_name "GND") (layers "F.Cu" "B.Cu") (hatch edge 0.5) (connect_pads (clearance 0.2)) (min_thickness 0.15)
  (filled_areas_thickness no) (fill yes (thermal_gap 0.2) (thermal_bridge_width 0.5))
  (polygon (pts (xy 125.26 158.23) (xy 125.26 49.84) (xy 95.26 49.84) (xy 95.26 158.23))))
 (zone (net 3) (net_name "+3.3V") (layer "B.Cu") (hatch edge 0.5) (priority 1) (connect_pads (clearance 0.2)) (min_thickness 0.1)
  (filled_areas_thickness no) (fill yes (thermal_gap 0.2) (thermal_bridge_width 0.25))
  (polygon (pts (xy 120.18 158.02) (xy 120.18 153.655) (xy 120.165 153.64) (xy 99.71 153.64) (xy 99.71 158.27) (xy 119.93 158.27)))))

